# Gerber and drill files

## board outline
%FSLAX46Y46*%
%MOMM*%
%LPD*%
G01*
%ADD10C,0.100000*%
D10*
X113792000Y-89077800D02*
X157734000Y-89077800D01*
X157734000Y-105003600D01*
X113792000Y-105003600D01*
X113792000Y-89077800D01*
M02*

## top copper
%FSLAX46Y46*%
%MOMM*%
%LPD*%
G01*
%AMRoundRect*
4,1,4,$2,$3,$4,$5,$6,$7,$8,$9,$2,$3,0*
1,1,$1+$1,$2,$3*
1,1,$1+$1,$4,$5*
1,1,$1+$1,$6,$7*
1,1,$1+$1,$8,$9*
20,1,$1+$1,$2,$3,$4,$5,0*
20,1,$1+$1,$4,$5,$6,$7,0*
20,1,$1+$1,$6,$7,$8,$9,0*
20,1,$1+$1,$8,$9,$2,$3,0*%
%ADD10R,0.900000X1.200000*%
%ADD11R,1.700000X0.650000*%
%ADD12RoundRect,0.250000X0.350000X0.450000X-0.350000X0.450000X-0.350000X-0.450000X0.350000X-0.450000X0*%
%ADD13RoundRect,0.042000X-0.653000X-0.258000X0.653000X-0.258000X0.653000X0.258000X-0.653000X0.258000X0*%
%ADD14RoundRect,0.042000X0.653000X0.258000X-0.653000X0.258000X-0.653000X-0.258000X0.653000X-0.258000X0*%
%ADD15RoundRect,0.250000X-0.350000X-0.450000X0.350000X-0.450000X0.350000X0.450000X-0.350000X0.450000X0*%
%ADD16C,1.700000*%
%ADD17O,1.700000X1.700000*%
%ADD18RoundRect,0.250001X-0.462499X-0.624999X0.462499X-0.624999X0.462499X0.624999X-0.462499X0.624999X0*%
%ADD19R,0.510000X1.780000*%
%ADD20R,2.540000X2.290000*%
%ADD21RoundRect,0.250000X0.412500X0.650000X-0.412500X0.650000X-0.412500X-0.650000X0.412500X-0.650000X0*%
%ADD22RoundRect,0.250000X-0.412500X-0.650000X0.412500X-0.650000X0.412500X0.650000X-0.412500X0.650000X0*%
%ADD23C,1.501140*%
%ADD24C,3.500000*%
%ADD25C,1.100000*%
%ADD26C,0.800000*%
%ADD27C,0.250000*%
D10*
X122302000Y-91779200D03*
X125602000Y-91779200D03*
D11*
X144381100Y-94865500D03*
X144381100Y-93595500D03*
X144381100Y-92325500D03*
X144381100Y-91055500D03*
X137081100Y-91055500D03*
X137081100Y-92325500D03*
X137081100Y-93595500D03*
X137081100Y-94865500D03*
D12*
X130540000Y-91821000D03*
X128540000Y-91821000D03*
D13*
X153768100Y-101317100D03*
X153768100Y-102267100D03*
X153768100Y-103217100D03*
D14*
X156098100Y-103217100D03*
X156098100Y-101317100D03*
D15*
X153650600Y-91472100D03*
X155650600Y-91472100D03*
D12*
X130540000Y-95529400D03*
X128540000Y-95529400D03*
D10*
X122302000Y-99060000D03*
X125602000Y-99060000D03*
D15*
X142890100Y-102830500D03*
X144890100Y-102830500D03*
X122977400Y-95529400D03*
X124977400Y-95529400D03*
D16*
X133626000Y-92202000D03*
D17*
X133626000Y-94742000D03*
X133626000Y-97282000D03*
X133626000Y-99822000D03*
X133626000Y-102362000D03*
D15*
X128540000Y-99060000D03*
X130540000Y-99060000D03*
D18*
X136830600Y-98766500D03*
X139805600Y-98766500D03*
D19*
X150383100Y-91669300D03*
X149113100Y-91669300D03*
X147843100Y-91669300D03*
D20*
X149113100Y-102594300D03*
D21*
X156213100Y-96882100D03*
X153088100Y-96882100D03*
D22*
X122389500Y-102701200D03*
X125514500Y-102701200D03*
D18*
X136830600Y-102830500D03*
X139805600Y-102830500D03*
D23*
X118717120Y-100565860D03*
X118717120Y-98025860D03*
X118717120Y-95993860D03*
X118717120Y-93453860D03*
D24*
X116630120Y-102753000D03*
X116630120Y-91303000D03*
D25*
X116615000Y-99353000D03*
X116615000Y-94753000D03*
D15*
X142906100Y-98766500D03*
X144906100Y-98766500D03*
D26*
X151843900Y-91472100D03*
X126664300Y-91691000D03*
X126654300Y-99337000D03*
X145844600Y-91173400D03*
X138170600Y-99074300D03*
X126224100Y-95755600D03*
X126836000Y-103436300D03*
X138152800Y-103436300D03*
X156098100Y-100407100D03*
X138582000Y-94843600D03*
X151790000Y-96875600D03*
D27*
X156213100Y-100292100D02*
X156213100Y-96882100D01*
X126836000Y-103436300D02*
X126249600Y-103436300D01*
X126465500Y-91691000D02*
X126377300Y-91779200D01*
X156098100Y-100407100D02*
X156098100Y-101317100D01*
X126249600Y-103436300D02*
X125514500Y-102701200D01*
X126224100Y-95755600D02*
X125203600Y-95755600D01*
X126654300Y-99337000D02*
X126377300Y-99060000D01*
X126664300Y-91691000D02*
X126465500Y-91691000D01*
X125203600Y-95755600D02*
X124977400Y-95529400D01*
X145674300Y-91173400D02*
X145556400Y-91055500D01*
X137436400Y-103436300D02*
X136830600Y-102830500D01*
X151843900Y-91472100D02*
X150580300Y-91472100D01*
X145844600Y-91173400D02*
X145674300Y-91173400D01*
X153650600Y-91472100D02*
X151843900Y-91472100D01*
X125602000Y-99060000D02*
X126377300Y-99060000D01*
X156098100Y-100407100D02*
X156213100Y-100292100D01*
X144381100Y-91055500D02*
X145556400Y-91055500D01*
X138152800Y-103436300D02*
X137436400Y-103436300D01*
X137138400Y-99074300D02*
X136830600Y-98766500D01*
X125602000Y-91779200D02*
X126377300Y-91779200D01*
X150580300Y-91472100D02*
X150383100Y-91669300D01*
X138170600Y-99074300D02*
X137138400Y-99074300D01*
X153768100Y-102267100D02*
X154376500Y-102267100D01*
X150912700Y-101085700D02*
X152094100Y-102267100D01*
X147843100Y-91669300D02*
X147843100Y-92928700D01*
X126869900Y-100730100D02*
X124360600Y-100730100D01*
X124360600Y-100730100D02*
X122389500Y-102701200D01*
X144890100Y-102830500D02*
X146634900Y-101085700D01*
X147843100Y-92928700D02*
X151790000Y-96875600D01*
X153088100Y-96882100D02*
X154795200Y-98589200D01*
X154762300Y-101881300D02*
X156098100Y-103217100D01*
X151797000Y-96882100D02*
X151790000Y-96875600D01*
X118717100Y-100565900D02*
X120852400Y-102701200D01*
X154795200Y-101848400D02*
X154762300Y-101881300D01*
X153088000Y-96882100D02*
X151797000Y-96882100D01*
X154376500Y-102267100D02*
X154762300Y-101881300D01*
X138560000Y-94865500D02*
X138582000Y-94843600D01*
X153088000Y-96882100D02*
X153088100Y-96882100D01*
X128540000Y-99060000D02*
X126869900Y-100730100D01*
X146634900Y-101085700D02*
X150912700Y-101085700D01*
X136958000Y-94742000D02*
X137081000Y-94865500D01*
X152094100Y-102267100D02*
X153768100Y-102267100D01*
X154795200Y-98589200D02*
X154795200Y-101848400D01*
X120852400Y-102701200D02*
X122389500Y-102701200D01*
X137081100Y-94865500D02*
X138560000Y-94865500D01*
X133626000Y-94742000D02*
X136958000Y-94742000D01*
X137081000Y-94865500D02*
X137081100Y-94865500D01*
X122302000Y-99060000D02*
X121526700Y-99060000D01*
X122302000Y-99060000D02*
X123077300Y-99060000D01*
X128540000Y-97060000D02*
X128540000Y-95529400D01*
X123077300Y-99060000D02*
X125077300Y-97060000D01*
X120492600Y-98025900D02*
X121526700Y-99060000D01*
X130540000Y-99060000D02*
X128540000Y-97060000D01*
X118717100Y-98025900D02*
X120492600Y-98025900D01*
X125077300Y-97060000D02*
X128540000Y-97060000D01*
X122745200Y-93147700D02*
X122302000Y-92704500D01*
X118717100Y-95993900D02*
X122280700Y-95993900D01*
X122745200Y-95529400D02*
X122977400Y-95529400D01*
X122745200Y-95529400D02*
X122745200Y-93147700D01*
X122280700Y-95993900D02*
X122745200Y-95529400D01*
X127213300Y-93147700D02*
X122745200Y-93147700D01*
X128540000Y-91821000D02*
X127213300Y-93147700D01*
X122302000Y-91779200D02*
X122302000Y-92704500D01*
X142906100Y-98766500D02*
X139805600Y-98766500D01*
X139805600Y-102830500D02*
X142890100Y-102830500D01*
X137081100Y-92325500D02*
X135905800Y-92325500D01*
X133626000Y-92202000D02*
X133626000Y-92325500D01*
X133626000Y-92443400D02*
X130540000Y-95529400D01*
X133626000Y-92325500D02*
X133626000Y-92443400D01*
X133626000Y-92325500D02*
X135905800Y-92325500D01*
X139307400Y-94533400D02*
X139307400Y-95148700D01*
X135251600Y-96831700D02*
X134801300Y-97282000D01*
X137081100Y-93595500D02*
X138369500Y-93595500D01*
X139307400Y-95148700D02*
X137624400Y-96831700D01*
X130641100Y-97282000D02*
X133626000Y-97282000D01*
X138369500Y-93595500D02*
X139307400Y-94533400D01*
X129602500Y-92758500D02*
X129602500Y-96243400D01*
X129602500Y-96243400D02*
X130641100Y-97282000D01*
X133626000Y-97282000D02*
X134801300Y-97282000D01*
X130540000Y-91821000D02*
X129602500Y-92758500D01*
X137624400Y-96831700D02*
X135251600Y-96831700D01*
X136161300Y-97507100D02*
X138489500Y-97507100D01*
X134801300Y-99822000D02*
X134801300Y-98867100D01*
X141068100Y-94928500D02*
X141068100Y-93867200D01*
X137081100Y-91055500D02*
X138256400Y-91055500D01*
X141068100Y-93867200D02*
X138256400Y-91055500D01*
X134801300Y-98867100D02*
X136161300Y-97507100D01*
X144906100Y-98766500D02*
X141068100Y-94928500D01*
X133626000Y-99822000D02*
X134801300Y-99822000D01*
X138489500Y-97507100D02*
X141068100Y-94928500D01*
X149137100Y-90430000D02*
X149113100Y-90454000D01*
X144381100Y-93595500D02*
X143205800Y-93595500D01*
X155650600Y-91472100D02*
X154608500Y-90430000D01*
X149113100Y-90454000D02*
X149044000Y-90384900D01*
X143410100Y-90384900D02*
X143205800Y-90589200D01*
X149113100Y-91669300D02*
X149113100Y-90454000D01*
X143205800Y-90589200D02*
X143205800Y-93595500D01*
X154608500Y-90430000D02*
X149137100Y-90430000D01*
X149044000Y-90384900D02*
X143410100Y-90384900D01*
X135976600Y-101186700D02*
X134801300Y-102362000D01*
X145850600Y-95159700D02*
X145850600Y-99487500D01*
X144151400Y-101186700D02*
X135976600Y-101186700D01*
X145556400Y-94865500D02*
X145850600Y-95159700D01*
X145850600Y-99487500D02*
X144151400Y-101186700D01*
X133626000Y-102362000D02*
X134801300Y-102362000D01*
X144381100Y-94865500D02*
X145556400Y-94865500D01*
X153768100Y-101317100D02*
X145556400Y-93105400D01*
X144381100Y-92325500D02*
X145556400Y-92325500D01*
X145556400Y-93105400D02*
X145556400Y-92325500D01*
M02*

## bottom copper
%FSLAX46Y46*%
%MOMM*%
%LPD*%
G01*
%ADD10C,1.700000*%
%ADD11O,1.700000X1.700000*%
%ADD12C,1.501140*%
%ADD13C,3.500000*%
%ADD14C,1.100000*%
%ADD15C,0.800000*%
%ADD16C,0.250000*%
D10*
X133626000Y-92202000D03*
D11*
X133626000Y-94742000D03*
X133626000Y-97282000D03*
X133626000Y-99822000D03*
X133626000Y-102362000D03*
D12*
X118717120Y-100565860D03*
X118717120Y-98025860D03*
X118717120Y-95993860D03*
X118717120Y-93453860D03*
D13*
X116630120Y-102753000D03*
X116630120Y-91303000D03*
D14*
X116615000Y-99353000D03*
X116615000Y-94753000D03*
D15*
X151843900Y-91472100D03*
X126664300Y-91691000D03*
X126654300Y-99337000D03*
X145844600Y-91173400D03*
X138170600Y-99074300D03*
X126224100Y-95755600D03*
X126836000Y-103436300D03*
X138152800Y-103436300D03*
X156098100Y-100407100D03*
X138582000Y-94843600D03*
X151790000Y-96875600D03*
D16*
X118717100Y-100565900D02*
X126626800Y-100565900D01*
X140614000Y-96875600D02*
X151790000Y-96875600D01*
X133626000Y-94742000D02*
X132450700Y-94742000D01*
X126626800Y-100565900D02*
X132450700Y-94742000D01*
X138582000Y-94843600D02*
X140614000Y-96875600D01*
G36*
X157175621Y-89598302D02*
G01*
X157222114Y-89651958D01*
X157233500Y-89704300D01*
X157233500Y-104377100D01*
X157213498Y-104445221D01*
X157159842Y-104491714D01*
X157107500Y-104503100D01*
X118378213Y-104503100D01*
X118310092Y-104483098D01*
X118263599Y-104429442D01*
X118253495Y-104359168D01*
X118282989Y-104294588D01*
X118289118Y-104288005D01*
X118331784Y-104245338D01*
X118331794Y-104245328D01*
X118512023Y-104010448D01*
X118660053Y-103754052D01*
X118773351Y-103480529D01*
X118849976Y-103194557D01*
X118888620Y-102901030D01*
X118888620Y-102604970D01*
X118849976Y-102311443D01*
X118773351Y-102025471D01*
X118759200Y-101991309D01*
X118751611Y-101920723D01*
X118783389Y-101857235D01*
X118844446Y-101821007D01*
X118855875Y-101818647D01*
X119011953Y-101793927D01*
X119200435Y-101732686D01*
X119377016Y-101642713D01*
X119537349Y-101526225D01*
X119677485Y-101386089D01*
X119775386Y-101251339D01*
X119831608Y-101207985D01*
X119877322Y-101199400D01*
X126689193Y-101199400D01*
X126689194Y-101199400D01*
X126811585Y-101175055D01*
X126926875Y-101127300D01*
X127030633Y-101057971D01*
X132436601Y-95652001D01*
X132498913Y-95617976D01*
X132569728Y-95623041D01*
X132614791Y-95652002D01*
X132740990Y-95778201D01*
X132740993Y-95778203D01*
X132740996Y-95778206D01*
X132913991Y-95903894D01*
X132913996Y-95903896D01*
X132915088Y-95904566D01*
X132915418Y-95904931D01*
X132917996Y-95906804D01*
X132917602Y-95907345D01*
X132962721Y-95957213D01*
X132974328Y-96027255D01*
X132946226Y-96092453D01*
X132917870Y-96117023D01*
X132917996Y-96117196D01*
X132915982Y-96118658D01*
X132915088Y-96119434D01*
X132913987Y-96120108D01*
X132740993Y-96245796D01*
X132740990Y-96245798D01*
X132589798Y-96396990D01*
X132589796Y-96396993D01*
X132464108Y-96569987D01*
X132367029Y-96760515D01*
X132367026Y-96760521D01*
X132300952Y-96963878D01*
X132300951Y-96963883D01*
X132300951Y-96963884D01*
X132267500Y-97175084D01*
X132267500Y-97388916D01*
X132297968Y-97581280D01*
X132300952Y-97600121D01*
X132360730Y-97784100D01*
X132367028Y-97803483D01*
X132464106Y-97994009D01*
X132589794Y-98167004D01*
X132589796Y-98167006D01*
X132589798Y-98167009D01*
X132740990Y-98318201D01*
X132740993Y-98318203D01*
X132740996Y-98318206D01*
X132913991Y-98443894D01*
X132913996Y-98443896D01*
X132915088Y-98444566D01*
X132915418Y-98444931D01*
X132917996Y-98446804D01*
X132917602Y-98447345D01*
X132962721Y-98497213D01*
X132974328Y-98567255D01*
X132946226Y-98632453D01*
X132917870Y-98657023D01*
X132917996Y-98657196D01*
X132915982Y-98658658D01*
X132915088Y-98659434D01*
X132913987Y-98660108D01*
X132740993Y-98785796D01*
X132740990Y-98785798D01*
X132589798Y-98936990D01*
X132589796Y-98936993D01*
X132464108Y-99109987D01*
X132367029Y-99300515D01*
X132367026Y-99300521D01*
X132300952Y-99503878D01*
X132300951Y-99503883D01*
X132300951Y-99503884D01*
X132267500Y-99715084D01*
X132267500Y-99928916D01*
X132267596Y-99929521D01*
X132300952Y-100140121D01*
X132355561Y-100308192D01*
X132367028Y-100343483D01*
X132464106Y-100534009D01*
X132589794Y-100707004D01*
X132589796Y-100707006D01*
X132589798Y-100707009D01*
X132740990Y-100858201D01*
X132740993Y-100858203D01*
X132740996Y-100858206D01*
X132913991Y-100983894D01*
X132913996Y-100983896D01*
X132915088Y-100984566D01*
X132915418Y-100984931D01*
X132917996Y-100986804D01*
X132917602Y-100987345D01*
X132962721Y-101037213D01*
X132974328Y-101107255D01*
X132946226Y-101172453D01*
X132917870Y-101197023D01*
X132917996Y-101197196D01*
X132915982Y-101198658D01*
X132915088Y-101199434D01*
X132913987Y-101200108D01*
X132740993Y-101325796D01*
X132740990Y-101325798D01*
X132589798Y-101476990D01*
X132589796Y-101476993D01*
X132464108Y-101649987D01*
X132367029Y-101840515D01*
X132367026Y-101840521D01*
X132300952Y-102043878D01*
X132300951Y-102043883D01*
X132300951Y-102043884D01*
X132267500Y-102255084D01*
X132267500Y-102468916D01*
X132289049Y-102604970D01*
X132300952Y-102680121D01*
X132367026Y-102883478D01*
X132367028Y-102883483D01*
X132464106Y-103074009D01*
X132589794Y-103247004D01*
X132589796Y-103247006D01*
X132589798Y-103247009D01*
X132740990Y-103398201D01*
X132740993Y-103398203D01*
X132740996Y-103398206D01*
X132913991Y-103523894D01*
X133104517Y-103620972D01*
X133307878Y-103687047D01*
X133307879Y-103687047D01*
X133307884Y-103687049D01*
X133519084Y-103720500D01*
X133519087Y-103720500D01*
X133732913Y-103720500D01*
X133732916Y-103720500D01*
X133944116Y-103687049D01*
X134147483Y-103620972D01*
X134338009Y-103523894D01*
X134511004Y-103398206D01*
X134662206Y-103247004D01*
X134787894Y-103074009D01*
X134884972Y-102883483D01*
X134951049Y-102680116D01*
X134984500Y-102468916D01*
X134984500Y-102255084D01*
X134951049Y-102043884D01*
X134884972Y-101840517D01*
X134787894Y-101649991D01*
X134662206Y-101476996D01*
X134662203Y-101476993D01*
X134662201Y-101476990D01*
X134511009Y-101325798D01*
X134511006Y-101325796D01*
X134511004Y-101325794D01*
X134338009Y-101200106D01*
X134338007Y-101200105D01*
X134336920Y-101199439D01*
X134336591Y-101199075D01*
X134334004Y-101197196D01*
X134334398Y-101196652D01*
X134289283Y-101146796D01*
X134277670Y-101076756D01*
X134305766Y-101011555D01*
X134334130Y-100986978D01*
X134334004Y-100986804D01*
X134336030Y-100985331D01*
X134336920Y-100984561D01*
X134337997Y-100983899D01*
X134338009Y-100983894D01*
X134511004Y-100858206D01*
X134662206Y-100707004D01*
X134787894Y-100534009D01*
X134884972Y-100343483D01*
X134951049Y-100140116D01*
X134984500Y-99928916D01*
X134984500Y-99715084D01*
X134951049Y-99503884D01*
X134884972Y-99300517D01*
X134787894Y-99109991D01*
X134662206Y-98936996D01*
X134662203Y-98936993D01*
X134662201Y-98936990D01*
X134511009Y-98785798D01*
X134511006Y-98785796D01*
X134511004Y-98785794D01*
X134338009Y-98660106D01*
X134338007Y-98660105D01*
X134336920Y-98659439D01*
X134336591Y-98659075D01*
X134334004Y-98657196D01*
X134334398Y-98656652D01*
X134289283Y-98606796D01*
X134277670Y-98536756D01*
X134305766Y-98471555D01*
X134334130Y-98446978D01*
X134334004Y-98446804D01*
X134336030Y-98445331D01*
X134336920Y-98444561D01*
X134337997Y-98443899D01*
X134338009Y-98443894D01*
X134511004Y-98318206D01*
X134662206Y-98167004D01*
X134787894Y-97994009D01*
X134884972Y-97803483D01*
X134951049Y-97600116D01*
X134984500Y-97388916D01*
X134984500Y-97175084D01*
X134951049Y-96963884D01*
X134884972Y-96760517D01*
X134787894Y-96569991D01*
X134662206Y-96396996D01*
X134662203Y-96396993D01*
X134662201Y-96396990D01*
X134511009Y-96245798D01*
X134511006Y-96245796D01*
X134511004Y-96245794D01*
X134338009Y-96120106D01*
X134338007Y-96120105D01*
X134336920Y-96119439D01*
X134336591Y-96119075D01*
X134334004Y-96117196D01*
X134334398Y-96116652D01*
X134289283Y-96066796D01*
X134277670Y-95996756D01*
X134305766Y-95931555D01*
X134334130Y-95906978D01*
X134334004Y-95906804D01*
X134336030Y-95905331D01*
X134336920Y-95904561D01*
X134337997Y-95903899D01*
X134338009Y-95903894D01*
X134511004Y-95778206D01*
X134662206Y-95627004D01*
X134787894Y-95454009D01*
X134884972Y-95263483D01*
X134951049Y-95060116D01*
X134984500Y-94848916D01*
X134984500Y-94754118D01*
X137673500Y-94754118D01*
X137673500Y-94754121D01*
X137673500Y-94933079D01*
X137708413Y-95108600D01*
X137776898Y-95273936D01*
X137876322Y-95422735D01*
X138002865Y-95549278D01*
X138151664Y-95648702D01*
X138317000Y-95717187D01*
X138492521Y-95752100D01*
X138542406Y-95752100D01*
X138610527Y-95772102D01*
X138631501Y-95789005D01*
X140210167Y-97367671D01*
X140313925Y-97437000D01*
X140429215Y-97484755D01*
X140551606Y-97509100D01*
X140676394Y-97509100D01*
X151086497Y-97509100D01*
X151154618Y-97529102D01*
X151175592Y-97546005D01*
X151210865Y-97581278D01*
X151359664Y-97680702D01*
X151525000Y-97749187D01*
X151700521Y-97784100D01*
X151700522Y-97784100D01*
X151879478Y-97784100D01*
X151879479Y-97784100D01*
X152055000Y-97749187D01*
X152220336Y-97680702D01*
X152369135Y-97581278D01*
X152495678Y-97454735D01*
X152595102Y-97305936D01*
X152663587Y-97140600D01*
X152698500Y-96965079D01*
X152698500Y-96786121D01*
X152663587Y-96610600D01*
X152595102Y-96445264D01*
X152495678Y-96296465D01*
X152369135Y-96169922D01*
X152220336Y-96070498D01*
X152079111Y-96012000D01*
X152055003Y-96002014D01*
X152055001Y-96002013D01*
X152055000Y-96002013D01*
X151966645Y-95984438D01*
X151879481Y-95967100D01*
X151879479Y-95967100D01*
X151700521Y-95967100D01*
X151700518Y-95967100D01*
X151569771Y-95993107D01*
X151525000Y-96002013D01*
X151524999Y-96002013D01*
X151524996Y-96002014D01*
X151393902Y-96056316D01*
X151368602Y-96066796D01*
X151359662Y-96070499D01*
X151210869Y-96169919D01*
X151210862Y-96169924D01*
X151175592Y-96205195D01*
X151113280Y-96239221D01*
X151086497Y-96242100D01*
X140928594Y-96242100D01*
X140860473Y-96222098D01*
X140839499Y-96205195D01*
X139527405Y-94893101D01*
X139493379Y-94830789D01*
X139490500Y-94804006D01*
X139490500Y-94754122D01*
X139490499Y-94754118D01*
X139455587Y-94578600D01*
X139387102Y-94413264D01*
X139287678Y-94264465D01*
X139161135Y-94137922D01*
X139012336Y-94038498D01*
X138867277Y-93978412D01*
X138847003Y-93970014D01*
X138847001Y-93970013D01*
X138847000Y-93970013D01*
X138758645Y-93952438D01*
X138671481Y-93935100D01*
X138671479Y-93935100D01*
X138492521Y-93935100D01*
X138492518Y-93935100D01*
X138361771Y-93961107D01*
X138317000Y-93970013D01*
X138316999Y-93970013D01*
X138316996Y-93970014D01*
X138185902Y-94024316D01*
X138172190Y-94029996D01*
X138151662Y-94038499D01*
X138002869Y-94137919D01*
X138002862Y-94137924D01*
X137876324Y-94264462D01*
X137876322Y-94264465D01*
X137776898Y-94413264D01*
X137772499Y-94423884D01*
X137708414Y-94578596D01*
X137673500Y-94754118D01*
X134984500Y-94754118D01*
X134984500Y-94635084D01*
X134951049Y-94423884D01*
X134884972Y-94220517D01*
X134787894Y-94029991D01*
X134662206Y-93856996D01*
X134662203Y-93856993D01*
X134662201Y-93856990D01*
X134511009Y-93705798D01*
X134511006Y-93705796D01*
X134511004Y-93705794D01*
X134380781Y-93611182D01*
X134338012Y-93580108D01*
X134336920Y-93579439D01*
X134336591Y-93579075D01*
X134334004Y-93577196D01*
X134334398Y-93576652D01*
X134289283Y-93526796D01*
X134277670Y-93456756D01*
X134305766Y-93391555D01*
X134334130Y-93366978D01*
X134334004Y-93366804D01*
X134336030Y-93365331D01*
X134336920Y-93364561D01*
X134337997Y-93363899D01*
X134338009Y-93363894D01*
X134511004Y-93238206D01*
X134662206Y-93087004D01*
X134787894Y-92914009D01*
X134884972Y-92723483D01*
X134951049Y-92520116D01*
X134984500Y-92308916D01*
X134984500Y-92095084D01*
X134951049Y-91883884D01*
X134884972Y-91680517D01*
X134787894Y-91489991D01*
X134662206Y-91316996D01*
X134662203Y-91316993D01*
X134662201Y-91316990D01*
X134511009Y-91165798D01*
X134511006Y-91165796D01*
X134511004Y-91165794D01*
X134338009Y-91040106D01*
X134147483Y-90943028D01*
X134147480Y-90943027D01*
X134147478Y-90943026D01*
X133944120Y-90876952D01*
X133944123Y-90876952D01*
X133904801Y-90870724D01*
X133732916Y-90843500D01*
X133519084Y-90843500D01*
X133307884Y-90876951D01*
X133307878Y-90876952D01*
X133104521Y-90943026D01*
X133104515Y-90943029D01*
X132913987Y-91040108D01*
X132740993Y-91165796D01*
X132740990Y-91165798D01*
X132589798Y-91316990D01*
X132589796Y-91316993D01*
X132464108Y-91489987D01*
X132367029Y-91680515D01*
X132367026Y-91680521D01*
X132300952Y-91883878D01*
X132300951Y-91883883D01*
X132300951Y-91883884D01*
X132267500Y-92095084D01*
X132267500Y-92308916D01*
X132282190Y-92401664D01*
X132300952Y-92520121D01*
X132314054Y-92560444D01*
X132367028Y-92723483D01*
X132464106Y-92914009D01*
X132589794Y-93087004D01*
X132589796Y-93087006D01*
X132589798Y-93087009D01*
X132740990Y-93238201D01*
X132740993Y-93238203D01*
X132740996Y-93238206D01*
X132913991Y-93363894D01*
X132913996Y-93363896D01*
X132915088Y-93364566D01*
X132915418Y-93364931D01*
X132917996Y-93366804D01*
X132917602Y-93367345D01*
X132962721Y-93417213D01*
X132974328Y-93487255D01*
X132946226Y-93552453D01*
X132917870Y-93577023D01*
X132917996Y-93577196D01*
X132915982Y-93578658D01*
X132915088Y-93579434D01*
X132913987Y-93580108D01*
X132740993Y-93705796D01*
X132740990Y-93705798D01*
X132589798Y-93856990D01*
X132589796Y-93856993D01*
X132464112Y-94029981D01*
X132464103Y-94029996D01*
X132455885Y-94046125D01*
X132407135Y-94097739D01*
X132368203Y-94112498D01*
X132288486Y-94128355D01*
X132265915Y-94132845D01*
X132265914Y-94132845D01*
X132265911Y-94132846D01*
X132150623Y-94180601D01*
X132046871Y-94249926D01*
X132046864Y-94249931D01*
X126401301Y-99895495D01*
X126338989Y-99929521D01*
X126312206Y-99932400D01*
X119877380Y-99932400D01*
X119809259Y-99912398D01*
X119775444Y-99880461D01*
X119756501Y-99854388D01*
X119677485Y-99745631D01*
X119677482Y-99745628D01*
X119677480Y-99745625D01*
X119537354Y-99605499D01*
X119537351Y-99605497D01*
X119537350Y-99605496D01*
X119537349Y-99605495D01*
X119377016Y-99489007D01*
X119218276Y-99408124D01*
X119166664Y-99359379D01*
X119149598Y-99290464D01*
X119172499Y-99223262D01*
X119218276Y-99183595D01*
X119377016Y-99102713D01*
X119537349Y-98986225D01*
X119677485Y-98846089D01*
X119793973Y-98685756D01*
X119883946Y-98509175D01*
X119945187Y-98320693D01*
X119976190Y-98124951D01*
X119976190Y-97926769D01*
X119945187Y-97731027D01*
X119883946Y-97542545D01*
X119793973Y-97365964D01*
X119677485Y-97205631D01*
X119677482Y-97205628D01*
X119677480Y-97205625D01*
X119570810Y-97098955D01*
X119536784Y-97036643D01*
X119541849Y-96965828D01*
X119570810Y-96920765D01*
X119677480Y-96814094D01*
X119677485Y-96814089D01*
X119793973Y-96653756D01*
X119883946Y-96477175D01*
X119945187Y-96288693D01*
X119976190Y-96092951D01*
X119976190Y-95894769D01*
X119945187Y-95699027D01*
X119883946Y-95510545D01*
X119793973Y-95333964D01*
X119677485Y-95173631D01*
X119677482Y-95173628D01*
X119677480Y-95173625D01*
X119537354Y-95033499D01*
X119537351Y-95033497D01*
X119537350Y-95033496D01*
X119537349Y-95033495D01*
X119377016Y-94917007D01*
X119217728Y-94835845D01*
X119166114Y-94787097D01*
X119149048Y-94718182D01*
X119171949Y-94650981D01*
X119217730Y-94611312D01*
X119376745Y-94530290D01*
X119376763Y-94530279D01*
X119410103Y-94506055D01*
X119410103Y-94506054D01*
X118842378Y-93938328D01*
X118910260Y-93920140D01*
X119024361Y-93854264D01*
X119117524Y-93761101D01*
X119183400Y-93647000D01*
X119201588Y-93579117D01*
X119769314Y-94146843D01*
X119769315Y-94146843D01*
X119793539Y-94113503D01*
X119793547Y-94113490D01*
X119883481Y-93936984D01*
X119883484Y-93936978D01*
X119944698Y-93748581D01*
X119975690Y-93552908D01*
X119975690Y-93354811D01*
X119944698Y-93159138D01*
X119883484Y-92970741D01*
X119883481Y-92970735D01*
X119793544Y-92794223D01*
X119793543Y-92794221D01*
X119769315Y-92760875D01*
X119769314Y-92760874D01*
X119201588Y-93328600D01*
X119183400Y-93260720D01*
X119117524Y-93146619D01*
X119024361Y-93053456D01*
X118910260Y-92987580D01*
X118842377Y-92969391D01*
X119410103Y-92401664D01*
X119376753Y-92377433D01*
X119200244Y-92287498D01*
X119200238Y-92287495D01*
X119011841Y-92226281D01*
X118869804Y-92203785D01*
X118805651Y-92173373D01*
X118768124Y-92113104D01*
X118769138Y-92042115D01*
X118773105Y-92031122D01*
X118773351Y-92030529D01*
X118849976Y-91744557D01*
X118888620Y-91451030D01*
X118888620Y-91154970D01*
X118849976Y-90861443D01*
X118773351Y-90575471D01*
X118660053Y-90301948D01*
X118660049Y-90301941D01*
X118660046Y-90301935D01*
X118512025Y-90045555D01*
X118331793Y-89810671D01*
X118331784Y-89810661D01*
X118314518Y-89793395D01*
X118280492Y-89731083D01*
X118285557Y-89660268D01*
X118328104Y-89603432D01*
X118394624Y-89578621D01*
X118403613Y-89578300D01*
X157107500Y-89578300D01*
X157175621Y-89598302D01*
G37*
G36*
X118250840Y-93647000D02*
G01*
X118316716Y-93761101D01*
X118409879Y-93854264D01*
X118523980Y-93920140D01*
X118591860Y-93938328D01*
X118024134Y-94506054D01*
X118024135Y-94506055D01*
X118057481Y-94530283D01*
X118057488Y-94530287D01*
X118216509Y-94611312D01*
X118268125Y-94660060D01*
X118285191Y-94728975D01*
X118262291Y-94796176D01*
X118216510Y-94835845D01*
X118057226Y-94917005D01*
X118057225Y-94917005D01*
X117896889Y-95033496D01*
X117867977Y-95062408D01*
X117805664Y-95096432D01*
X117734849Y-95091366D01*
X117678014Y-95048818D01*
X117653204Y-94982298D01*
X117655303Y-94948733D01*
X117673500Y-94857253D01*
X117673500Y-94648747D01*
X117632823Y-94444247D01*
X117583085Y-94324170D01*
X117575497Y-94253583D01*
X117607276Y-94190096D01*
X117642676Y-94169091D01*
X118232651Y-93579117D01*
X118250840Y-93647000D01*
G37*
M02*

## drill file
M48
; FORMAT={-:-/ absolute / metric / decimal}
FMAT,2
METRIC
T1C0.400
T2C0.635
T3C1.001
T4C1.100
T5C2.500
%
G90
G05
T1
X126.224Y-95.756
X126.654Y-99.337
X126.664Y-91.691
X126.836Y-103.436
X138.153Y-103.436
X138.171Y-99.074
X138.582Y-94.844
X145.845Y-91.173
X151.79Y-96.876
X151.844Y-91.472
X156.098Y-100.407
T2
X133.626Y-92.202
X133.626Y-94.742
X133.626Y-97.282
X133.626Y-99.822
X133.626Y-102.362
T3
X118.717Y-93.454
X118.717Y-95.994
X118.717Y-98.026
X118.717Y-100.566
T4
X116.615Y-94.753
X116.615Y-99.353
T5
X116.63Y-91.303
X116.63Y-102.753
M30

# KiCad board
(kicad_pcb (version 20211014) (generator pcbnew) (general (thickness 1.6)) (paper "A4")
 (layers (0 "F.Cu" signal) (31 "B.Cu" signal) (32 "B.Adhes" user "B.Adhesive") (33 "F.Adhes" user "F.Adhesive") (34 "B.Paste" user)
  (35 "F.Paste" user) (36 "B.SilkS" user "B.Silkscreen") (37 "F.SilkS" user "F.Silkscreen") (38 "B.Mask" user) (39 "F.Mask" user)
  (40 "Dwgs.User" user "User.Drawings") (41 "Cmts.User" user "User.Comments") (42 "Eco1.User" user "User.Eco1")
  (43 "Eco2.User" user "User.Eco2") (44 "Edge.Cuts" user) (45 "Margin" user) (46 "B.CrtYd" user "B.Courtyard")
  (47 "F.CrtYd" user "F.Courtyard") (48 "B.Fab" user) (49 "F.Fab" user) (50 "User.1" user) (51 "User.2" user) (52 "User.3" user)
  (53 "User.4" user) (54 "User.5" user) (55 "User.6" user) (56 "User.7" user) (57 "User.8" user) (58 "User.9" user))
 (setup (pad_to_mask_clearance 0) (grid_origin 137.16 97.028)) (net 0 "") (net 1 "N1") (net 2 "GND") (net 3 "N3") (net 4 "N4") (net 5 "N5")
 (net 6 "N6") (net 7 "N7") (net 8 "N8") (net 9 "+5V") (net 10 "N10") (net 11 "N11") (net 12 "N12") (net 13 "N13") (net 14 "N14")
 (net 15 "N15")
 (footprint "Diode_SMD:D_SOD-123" (layer "F.Cu") (at 123.952 91.7792)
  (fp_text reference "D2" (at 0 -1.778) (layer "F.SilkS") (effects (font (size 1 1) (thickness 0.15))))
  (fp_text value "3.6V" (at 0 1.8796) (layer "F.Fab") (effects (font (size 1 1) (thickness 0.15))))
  (pad "1" smd rect (at -1.65 0) (size 0.9 1.2) (layers "F.Cu" "F.Paste" "F.Mask") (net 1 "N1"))
  (pad "2" smd rect (at 1.65 0) (size 0.9 1.2) (layers "F.Cu" "F.Paste" "F.Mask") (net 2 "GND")))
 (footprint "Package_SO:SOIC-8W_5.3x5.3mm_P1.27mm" (layer "F.Cu") (at 140.7311 92.9605 180)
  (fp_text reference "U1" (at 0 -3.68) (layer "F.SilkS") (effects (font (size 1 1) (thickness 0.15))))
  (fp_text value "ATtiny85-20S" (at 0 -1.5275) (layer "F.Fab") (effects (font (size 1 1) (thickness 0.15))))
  (pad "1" smd rect (at -3.65 -1.905 180) (size 1.7 0.65) (layers "F.Cu" "F.Paste" "F.Mask") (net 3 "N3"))
  (pad "2" smd rect (at -3.65 -0.635 180) (size 1.7 0.65) (layers "F.Cu" "F.Paste" "F.Mask") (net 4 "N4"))
  (pad "3" smd rect (at -3.65 0.635 180) (size 1.7 0.65) (layers "F.Cu" "F.Paste" "F.Mask") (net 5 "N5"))
  (pad "4" smd rect (at -3.65 1.905 180) (size 1.7 0.65) (layers "F.Cu" "F.Paste" "F.Mask") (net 2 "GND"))
  (pad "5" smd rect (at 3.65 1.905 180) (size 1.7 0.65) (layers "F.Cu" "F.Paste" "F.Mask") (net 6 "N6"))
  (pad "6" smd rect (at 3.65 0.635 180) (size 1.7 0.65) (layers "F.Cu" "F.Paste" "F.Mask") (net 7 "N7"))
  (pad "7" smd rect (at 3.65 -0.635 180) (size 1.7 0.65) (layers "F.Cu" "F.Paste" "F.Mask") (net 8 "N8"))
  (pad "8" smd rect (at 3.65 -1.905 180) (size 1.7 0.65) (layers "F.Cu" "F.Paste" "F.Mask") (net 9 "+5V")))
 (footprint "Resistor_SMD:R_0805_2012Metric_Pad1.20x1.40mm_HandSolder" (layer "F.Cu") (at 129.54 91.821 180)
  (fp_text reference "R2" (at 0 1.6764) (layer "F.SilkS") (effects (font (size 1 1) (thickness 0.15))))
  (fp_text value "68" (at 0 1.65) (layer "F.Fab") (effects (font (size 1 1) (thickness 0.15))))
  (pad "1" smd roundrect (at -1 0 180) (size 1.2 1.4) (layers "F.Cu" "F.Paste" "F.Mask") (roundrect_rratio 0.208333) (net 8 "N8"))
  (pad "2" smd roundrect (at 1 0 180) (size 1.2 1.4) (layers "F.Cu" "F.Paste" "F.Mask") (roundrect_rratio 0.208333) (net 1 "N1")))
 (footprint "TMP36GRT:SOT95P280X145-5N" (layer "F.Cu") (at 154.9331 102.2671)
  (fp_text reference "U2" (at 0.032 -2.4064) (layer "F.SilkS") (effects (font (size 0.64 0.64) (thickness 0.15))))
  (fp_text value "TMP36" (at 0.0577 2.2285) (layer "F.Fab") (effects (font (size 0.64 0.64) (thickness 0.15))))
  (pad "1" smd roundrect locked (at -1.165 -0.95) (size 1.39 0.6) (layers "F.Cu" "F.Paste" "F.Mask") (roundrect_rratio 0.07) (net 5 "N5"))
  (pad "2" smd roundrect locked (at -1.165 0) (size 1.39 0.6) (layers "F.Cu" "F.Paste" "F.Mask") (roundrect_rratio 0.07) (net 9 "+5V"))
  (pad "3" smd roundrect locked (at -1.165 0.95) (size 1.39 0.6) (layers "F.Cu" "F.Paste" "F.Mask") (roundrect_rratio 0.07))
  (pad "4" smd roundrect locked (at 1.165 0.95 180) (size 1.39 0.6) (layers "F.Cu" "F.Paste" "F.Mask") (roundrect_rratio 0.07) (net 9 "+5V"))
  (pad "5" smd roundrect locked (at 1.165 -0.95 180) (size 1.39 0.6) (layers "F.Cu" "F.Paste" "F.Mask") (roundrect_rratio 0.07)
   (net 2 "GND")))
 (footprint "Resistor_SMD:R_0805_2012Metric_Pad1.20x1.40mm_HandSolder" (layer "F.Cu") (at 154.6506 91.4721)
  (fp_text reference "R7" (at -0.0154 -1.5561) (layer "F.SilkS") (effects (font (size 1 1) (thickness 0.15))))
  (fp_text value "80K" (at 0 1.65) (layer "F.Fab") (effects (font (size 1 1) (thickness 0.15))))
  (pad "1" smd roundrect (at -1 0) (size 1.2 1.4) (layers "F.Cu" "F.Paste" "F.Mask") (roundrect_rratio 0.208333) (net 2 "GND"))
  (pad "2" smd roundrect (at 1 0) (size 1.2 1.4) (layers "F.Cu" "F.Paste" "F.Mask") (roundrect_rratio 0.208333) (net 4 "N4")))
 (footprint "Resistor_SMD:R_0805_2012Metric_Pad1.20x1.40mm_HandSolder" (layer "F.Cu") (at 129.54 95.5294 180)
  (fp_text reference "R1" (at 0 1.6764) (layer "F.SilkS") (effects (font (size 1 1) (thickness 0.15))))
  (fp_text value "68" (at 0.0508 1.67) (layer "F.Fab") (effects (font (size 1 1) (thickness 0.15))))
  (pad "1" smd roundrect (at -1 0 180) (size 1.2 1.4) (layers "F.Cu" "F.Paste" "F.Mask") (roundrect_rratio 0.208333) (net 7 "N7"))
  (pad "2" smd roundrect (at 1 0 180) (size 1.2 1.4) (layers "F.Cu" "F.Paste" "F.Mask") (roundrect_rratio 0.208333) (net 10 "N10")))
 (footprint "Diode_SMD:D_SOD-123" (layer "F.Cu") (at 123.952 99.06)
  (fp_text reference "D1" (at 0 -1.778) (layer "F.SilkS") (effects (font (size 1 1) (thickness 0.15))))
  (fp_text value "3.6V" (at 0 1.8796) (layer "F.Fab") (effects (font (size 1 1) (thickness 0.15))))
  (pad "1" smd rect (at -1.65 0) (size 0.9 1.2) (layers "F.Cu" "F.Paste" "F.Mask") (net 10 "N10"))
  (pad "2" smd rect (at 1.65 0) (size 0.9 1.2) (layers "F.Cu" "F.Paste" "F.Mask") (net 2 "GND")))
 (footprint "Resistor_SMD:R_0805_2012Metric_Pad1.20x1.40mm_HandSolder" (layer "F.Cu") (at 143.8901 102.8305)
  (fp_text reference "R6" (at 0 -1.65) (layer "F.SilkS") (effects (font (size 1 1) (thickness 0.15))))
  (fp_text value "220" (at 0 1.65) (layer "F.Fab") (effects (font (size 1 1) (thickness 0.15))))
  (pad "1" smd roundrect (at -1 0) (size 1.2 1.4) (layers "F.Cu" "F.Paste" "F.Mask") (roundrect_rratio 0.208333) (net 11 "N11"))
  (pad "2" smd roundrect (at 1 0) (size 1.2 1.4) (layers "F.Cu" "F.Paste" "F.Mask") (roundrect_rratio 0.208333) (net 9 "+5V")))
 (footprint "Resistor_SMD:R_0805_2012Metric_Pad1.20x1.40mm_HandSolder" (layer "F.Cu") (at 123.9774 95.5294)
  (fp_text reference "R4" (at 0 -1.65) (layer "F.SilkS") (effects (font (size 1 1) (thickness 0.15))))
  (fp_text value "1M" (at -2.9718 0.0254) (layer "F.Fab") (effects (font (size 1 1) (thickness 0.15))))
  (pad "1" smd roundrect (at -1 0) (size 1.2 1.4) (layers "F.Cu" "F.Paste" "F.Mask") (roundrect_rratio 0.208333) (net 1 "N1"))
  (pad "2" smd roundrect (at 1 0) (size 1.2 1.4) (layers "F.Cu" "F.Paste" "F.Mask") (roundrect_rratio 0.208333) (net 2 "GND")))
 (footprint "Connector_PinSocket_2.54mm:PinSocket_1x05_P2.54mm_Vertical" (layer "F.Cu") (at 133.626 92.202)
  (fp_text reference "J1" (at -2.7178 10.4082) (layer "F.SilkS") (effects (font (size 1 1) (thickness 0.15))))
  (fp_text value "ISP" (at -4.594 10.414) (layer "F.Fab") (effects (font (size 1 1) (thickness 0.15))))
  (pad "1" thru_hole circle (at 0 0) (size 1.7 1.7) (drill 0.635) (layers *.Cu *.Mask) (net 7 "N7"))
  (pad "2" thru_hole oval (at 0 2.54) (size 1.7 1.7) (drill 0.635) (layers *.Cu *.Mask) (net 9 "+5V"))
  (pad "3" thru_hole oval (at 0 5.08) (size 1.7 1.7) (drill 0.635) (layers *.Cu *.Mask) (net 8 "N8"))
  (pad "4" thru_hole oval (at 0 7.62) (size 1.7 1.7) (drill 0.635) (layers *.Cu *.Mask) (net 6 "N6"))
  (pad "5" thru_hole oval (at 0 10.16) (size 1.7 1.7) (drill 0.635) (layers *.Cu *.Mask) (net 3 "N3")))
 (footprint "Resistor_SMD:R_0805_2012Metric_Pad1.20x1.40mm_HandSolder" (layer "F.Cu") (at 129.54 99.06)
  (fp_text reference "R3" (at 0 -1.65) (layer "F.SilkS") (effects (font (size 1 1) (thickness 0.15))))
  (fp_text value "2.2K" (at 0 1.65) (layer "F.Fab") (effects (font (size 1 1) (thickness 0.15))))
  (pad "1" smd roundrect (at -1 0) (size 1.2 1.4) (layers "F.Cu" "F.Paste" "F.Mask") (roundrect_rratio 0.208333) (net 9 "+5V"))
  (pad "2" smd roundrect (at 1 0) (size 1.2 1.4) (layers "F.Cu" "F.Paste" "F.Mask") (roundrect_rratio 0.208333) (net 10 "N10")))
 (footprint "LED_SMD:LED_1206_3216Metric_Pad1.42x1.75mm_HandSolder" (layer "F.Cu") (at 138.3181 98.7665)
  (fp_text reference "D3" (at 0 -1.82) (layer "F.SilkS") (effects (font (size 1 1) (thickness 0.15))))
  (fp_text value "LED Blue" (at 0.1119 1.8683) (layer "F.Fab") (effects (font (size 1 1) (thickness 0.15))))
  (pad "1" smd roundrect (at -1.4875 0) (size 1.425 1.75) (layers "F.Cu" "F.Paste" "F.Mask") (roundrect_rratio 0.175439) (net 2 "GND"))
  (pad "2" smd roundrect (at 1.4875 0) (size 1.425 1.75) (layers "F.Cu" "F.Paste" "F.Mask") (roundrect_rratio 0.175439) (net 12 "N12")))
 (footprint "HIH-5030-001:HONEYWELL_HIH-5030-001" (layer "F.Cu") (at 149.1131 97.0043 180)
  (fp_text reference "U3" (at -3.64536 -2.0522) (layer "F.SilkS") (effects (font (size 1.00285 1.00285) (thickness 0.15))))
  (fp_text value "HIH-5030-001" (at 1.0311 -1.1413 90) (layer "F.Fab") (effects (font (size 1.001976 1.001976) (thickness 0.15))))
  (pad "1" smd rect locked (at -1.27 5.335 270) (size 1.78 0.51) (layers "F.Cu" "F.Paste" "F.Mask") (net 2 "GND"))
  (pad "2" smd rect locked (at 0 5.335 270) (size 1.78 0.51) (layers "F.Cu" "F.Paste" "F.Mask") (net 4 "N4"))
  (pad "3" smd rect locked (at 1.27 5.335 270) (size 1.78 0.51) (layers "F.Cu" "F.Paste" "F.Mask") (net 9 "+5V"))
  (pad "4" smd rect locked (at 0 -5.59 180) (size 2.54 2.29) (layers "F.Cu" "F.Paste" "F.Mask") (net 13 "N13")))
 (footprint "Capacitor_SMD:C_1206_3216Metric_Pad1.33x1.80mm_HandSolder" (layer "F.Cu") (at 154.6506 96.8821 180)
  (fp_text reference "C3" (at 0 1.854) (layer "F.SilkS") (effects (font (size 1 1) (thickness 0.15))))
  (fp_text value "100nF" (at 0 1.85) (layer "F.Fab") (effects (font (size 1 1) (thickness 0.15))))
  (pad "1" smd roundrect (at -1.5625 0 180) (size 1.325 1.8) (layers "F.Cu" "F.Paste" "F.Mask") (roundrect_rratio 0.188679) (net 2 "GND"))
  (pad "2" smd roundrect (at 1.5625 0 180) (size 1.325 1.8) (layers "F.Cu" "F.Paste" "F.Mask") (roundrect_rratio 0.188679) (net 9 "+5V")))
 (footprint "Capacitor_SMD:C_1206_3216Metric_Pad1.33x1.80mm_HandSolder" (layer "F.Cu") (at 123.952 102.7012)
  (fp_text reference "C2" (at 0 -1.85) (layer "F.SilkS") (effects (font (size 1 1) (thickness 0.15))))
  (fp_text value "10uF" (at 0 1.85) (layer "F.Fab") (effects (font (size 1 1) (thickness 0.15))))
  (pad "1" smd roundrect (at -1.5625 0) (size 1.325 1.8) (layers "F.Cu" "F.Paste" "F.Mask") (roundrect_rratio 0.188679) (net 9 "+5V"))
  (pad "2" smd roundrect (at 1.5625 0) (size 1.325 1.8) (layers "F.Cu" "F.Paste" "F.Mask") (roundrect_rratio 0.188679) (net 2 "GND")))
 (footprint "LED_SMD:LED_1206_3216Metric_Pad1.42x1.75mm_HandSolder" (layer "F.Cu") (at 138.3181 102.8305)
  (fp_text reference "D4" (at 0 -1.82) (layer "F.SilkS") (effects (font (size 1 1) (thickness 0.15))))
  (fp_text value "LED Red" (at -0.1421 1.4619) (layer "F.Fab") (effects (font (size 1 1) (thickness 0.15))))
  (pad "1" smd roundrect (at -1.4875 0) (size 1.425 1.75) (layers "F.Cu" "F.Paste" "F.Mask") (roundrect_rratio 0.175439) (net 2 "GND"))
  (pad "2" smd roundrect (at 1.4875 0) (size 1.425 1.75) (layers "F.Cu" "F.Paste" "F.Mask") (roundrect_rratio 0.175439) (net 11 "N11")))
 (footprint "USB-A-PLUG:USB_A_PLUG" (layer "F.Cu") (at 118.715 93.453 -90)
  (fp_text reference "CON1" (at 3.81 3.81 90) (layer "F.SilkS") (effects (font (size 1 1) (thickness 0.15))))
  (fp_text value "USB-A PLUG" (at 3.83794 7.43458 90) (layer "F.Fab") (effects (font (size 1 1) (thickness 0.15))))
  (pad "1" thru_hole circle (at 7.11286 -0.00212 180) (size 1.50114 1.50114) (drill 1.00076) (layers *.Cu *.Mask "F.SilkS") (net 9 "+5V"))
  (pad "2" thru_hole circle (at 4.57286 -0.00212 180) (size 1.50114 1.50114) (drill 1.00076) (layers *.Cu *.Mask "F.SilkS") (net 10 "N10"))
  (pad "3" thru_hole circle (at 2.54086 -0.00212 180) (size 1.50114 1.50114) (drill 1.00076) (layers *.Cu *.Mask "F.SilkS") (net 1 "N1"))
  (pad "4" thru_hole circle (at 0.00086 -0.00212 180) (size 1.50114 1.50114) (drill 1.00076) (layers *.Cu *.Mask "F.SilkS") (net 2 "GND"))
  (pad "5" thru_hole circle (at 9.3 2.08488 180) (size 3.5 3.5) (drill 2.5) (layers *.Cu *.Mask "F.SilkS") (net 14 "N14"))
  (pad "6" thru_hole circle (at -2.15 2.08488 180) (size 3.5 3.5) (drill 2.5) (layers *.Cu *.Mask "F.SilkS") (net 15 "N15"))
  (pad "7" thru_hole circle (at 5.9 2.1 180) (size 1.1 1.1) (drill 1.1) (layers *.Cu *.Mask "F.SilkS"))
  (pad "8" thru_hole circle (at 1.3 2.1 180) (size 1.1 1.1) (drill 1.1) (layers *.Cu *.Mask "F.SilkS")))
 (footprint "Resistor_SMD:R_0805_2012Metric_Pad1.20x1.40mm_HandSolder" (layer "F.Cu") (at 143.9061 98.7665)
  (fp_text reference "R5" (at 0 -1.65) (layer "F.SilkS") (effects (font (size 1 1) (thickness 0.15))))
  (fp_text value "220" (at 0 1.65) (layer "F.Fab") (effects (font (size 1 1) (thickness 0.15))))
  (pad "1" smd roundrect (at -1 0) (size 1.2 1.4) (layers "F.Cu" "F.Paste" "F.Mask") (roundrect_rratio 0.208333) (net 12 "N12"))
  (pad "2" smd roundrect (at 1 0) (size 1.2 1.4) (layers "F.Cu" "F.Paste" "F.Mask") (roundrect_rratio 0.208333) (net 6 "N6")))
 (gr_rect (start 113.792 89.0778) (end 157.734 105.0036) (layer "Edge.Cuts") (width 0.1) (fill none))
 (segment (start 156.2131 100.2921) (end 156.2131 96.8821) (width 0.25) (layer "F.Cu") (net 2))
 (segment (start 126.836 103.4363) (end 126.2496 103.4363) (width 0.25) (layer "F.Cu") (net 2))
 (segment (start 126.4655 91.691) (end 126.3773 91.7792) (width 0.25) (layer "F.Cu") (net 2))
 (segment (start 156.0981 100.4071) (end 156.0981 101.3171) (width 0.25) (layer "F.Cu") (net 2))
 (segment (start 126.2496 103.4363) (end 125.5145 102.7012) (width 0.25) (layer "F.Cu") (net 2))
 (segment (start 126.2241 95.7556) (end 125.2036 95.7556) (width 0.25) (layer "F.Cu") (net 2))
 (segment (start 126.6543 99.337) (end 126.3773 99.06) (width 0.25) (layer "F.Cu") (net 2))
 (segment (start 126.6643 91.691) (end 126.4655 91.691) (width 0.25) (layer "F.Cu") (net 2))
 (segment (start 125.2036 95.7556) (end 124.9774 95.5294) (width 0.25) (layer "F.Cu") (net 2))
 (segment (start 145.6743 91.1734) (end 145.5564 91.0555) (width 0.25) (layer "F.Cu") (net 2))
 (segment (start 137.4364 103.4363) (end 136.8306 102.8305) (width 0.25) (layer "F.Cu") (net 2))
 (segment (start 151.8439 91.4721) (end 150.5803 91.4721) (width 0.25) (layer "F.Cu") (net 2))
 (segment (start 145.8446 91.1734) (end 145.6743 91.1734) (width 0.25) (layer "F.Cu") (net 2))
 (segment (start 153.6506 91.4721) (end 151.8439 91.4721) (width 0.25) (layer "F.Cu") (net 2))
 (segment (start 125.602 99.06) (end 126.3773 99.06) (width 0.25) (layer "F.Cu") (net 2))
 (segment (start 156.0981 100.4071) (end 156.2131 100.2921) (width 0.25) (layer "F.Cu") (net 2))
 (segment (start 144.3811 91.0555) (end 145.5564 91.0555) (width 0.25) (layer "F.Cu") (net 2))
 (segment (start 138.1528 103.4363) (end 137.4364 103.4363) (width 0.25) (layer "F.Cu") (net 2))
 (segment (start 137.1384 99.0743) (end 136.8306 98.7665) (width 0.25) (layer "F.Cu") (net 2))
 (segment (start 125.602 91.7792) (end 126.3773 91.7792) (width 0.25) (layer "F.Cu") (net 2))
 (segment (start 150.5803 91.4721) (end 150.3831 91.6693) (width 0.25) (layer "F.Cu") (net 2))
 (segment (start 138.1706 99.0743) (end 137.1384 99.0743) (width 0.25) (layer "F.Cu") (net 2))
 (via (at 151.8439 91.4721) (size 0.8) (drill 0.4) (layers "F.Cu" "B.Cu") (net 2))
 (via (at 126.6643 91.691) (size 0.8) (drill 0.4) (layers "F.Cu" "B.Cu") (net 2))
 (via (at 126.6543 99.337) (size 0.8) (drill 0.4) (layers "F.Cu" "B.Cu") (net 2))
 (via (at 145.8446 91.1734) (size 0.8) (drill 0.4) (layers "F.Cu" "B.Cu") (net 2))
 (via (at 138.1706 99.0743) (size 0.8) (drill 0.4) (layers "F.Cu" "B.Cu") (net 2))
 (via (at 126.2241 95.7556) (size 0.8) (drill 0.4) (layers "F.Cu" "B.Cu") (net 2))
 (via (at 126.836 103.4363) (size 0.8) (drill 0.4) (layers "F.Cu" "B.Cu") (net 2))
 (via (at 138.1528 103.4363) (size 0.8) (drill 0.4) (layers "F.Cu" "B.Cu") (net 2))
 (via (at 156.0981 100.4071) (size 0.8) (drill 0.4) (layers "F.Cu" "B.Cu") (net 2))
 (segment (start 153.7681 102.2671) (end 154.3765 102.2671) (width 0.25) (layer "F.Cu") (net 9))
 (segment (start 150.9127 101.0857) (end 152.0941 102.2671) (width 0.25) (layer "F.Cu") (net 9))
 (segment (start 147.8431 91.6693) (end 147.8431 92.9287) (width 0.25) (layer "F.Cu") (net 9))
 (segment (start 126.8699 100.7301) (end 124.3606 100.7301) (width 0.25) (layer "F.Cu") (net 9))
 (segment (start 124.3606 100.7301) (end 122.3895 102.7012) (width 0.25) (layer "F.Cu") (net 9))
 (segment (start 144.8901 102.8305) (end 146.6349 101.0857) (width 0.25) (layer "F.Cu") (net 9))
 (segment (start 147.8431 92.9287) (end 151.79 96.8756) (width 0.25) (layer "F.Cu") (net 9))
 (segment (start 153.0881 96.8821) (end 154.7952 98.5892) (width 0.25) (layer "F.Cu") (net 9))
 (segment (start 154.7623 101.8813) (end 156.0981 103.2171) (width 0.25) (layer "F.Cu") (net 9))
 (segment (start 151.797 96.8821) (end 151.79 96.8756) (width 0.25) (layer "F.Cu") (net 9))
 (segment (start 118.7171 100.5659) (end 120.8524 102.7012) (width 0.25) (layer "F.Cu") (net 9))
 (segment (start 154.7952 101.8484) (end 154.7623 101.8813) (width 0.25) (layer "F.Cu") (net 9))
 (segment (start 153.088 96.8821) (end 151.797 96.8821) (width 0.25) (layer "F.Cu") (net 9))
 (segment (start 154.3765 102.2671) (end 154.7623 101.8813) (width 0.25) (layer "F.Cu") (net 9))
 (segment (start 138.56 94.8655) (end 138.582 94.8436) (width 0.25) (layer "F.Cu") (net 9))
 (segment (start 153.088 96.8821) (end 153.0881 96.8821) (width 0.25) (layer "F.Cu") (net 9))
 (segment (start 128.54 99.06) (end 126.8699 100.7301) (width 0.25) (layer "F.Cu") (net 9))
 (segment (start 146.6349 101.0857) (end 150.9127 101.0857) (width 0.25) (layer "F.Cu") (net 9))
 (segment (start 136.958 94.742) (end 137.081 94.8655) (width 0.25) (layer "F.Cu") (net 9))
 (segment (start 152.0941 102.2671) (end 153.7681 102.2671) (width 0.25) (layer "F.Cu") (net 9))
 (segment (start 154.7952 98.5892) (end 154.7952 101.8484) (width 0.25) (layer "F.Cu") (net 9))
 (segment (start 120.8524 102.7012) (end 122.3895 102.7012) (width 0.25) (layer "F.Cu") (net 9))
 (segment (start 137.0811 94.8655) (end 138.56 94.8655) (width 0.25) (layer "F.Cu") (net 9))
 (segment (start 133.626 94.742) (end 136.958 94.742) (width 0.25) (layer "F.Cu") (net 9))
 (segment (start 137.081 94.8655) (end 137.0811 94.8655) (width 0.25) (layer "F.Cu") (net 9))
 (via (at 138.582 94.8436) (size 0.8) (drill 0.4) (layers "F.Cu" "B.Cu") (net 9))
 (via (at 151.79 96.8756) (size 0.8) (drill 0.4) (layers "F.Cu" "B.Cu") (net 9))
 (segment (start 118.7171 100.5659) (end 126.6268 100.5659) (width 0.25) (layer "B.Cu") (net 9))
 (segment (start 140.614 96.8756) (end 151.79 96.8756) (width 0.25) (layer "B.Cu") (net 9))
 (segment (start 133.626 94.742) (end 132.4507 94.742) (width 0.25) (layer "B.Cu") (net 9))
 (segment (start 126.6268 100.5659) (end 132.4507 94.742) (width 0.25) (layer "B.Cu") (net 9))
 (segment (start 138.582 94.8436) (end 140.614 96.8756) (width 0.25) (layer "B.Cu") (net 9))
 (segment (start 122.302 99.06) (end 121.5267 99.06) (width 0.25) (layer "F.Cu") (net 10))
 (segment (start 122.302 99.06) (end 123.0773 99.06) (width 0.25) (layer "F.Cu") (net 10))
 (segment (start 128.54 97.06) (end 128.54 95.5294) (width 0.25) (layer "F.Cu") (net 10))
 (segment (start 123.0773 99.06) (end 125.0773 97.06) (width 0.25) (layer "F.Cu") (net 10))
 (segment (start 120.4926 98.0259) (end 121.5267 99.06) (width 0.25) (layer "F.Cu") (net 10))
 (segment (start 130.54 99.06) (end 128.54 97.06) (width 0.25) (layer "F.Cu") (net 10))
 (segment (start 118.7171 98.0259) (end 120.4926 98.0259) (width 0.25) (layer "F.Cu") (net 10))
 (segment (start 125.0773 97.06) (end 128.54 97.06) (width 0.25) (layer "F.Cu") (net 10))
 (segment (start 122.7452 93.1477) (end 122.302 92.7045) (width 0.25) (layer "F.Cu") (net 1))
 (segment (start 118.7171 95.9939) (end 122.2807 95.9939) (width 0.25) (layer "F.Cu") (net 1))
 (segment (start 122.7452 95.5294) (end 122.9774 95.5294) (width 0.25) (layer "F.Cu") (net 1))
 (segment (start 122.7452 95.5294) (end 122.7452 93.1477) (width 0.25) (layer "F.Cu") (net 1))
 (segment (start 122.2807 95.9939) (end 122.7452 95.5294) (width 0.25) (layer "F.Cu") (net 1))
 (segment (start 127.2133 93.1477) (end 122.7452 93.1477) (width 0.25) (layer "F.Cu") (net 1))
 (segment (start 128.54 91.821) (end 127.2133 93.1477) (width 0.25) (layer "F.Cu") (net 1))
 (segment (start 122.302 91.7792) (end 122.302 92.7045) (width 0.25) (layer "F.Cu") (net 1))
 (segment (start 142.9061 98.7665) (end 139.8056 98.7665) (width 0.25) (layer "F.Cu") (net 12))
 (segment (start 139.8056 102.8305) (end 142.8901 102.8305) (width 0.25) (layer "F.Cu") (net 11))
 (segment (start 137.0811 92.3255) (end 135.9058 92.3255) (width 0.25) (layer "F.Cu") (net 7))
 (segment (start 133.626 92.202) (end 133.626 92.3255) (width 0.25) (layer "F.Cu") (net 7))
 (segment (start 133.626 92.4434) (end 130.54 95.5294) (width 0.25) (layer "F.Cu") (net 7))
 (segment (start 133.626 92.3255) (end 133.626 92.4434) (width 0.25) (layer "F.Cu") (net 7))
 (segment (start 133.626 92.3255) (end 135.9058 92.3255) (width 0.25) (layer "F.Cu") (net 7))
 (segment (start 139.3074 94.5334) (end 139.3074 95.1487) (width 0.25) (layer "F.Cu") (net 8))
 (segment (start 135.2516 96.8317) (end 134.8013 97.282) (width 0.25) (layer "F.Cu") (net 8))
 (segment (start 137.0811 93.5955) (end 138.3695 93.5955) (width 0.25) (layer "F.Cu") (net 8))
 (segment (start 139.3074 95.1487) (end 137.6244 96.8317) (width 0.25) (layer "F.Cu") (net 8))
 (segment (start 130.6411 97.282) (end 133.626 97.282) (width 0.25) (layer "F.Cu") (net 8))
 (segment (start 138.3695 93.5955) (end 139.3074 94.5334) (width 0.25) (layer "F.Cu") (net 8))
 (segment (start 129.6025 92.7585) (end 129.6025 96.2434) (width 0.25) (layer "F.Cu") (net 8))
 (segment (start 129.6025 96.2434) (end 130.6411 97.282) (width 0.25) (layer "F.Cu") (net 8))
 (segment (start 133.626 97.282) (end 134.8013 97.282) (width 0.25) (layer "F.Cu") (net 8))
 (segment (start 130.54 91.821) (end 129.6025 92.7585) (width 0.25) (layer "F.Cu") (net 8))
 (segment (start 137.6244 96.8317) (end 135.2516 96.8317) (width 0.25) (layer "F.Cu") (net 8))
 (segment (start 136.1613 97.5071) (end 138.4895 97.5071) (width 0.25) (layer "F.Cu") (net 6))
 (segment (start 134.8013 99.822) (end 134.8013 98.8671) (width 0.25) (layer "F.Cu") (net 6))
 (segment (start 141.0681 94.9285) (end 141.0681 93.8672) (width 0.25) (layer "F.Cu") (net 6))
 (segment (start 137.0811 91.0555) (end 138.2564 91.0555) (width 0.25) (layer "F.Cu") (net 6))
 (segment (start 141.0681 93.8672) (end 138.2564 91.0555) (width 0.25) (layer "F.Cu") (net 6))
 (segment (start 134.8013 98.8671) (end 136.1613 97.5071) (width 0.25) (layer "F.Cu") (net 6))
 (segment (start 144.9061 98.7665) (end 141.0681 94.9285) (width 0.25) (layer "F.Cu") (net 6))
 (segment (start 133.626 99.822) (end 134.8013 99.822) (width 0.25) (layer "F.Cu") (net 6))
 (segment (start 138.4895 97.5071) (end 141.0681 94.9285) (width 0.25) (layer "F.Cu") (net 6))
 (segment (start 149.1371 90.43) (end 149.1131 90.454) (width 0.25) (layer "F.Cu") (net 4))
 (segment (start 144.3811 93.5955) (end 143.2058 93.5955) (width 0.25) (layer "F.Cu") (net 4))
 (segment (start 155.6506 91.4721) (end 154.6085 90.43) (width 0.25) (layer "F.Cu") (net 4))
 (segment (start 149.1131 90.454) (end 149.044 90.3849) (width 0.25) (layer "F.Cu") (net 4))
 (segment (start 143.4101 90.3849) (end 143.2058 90.5892) (width 0.25) (layer "F.Cu") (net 4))
 (segment (start 149.1131 91.6693) (end 149.1131 90.454) (width 0.25) (layer "F.Cu") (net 4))
 (segment (start 143.2058 90.5892) (end 143.2058 93.5955) (width 0.25) (layer "F.Cu") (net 4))
 (segment (start 154.6085 90.43) (end 149.1371 90.43) (width 0.25) (layer "F.Cu") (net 4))
 (segment (start 149.044 90.3849) (end 143.4101 90.3849) (width 0.25) (layer "F.Cu") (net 4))
 (segment (start 135.9766 101.1867) (end 134.8013 102.362) (width 0.25) (layer "F.Cu") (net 3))
 (segment (start 145.8506 95.1597) (end 145.8506 99.4875) (width 0.25) (layer "F.Cu") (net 3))
 (segment (start 144.1514 101.1867) (end 135.9766 101.1867) (width 0.25) (layer "F.Cu") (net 3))
 (segment (start 145.5564 94.8655) (end 145.8506 95.1597) (width 0.25) (layer "F.Cu") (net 3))
 (segment (start 145.8506 99.4875) (end 144.1514 101.1867) (width 0.25) (layer "F.Cu") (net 3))
 (segment (start 133.626 102.362) (end 134.8013 102.362) (width 0.25) (layer "F.Cu") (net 3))
 (segment (start 144.3811 94.8655) (end 145.5564 94.8655) (width 0.25) (layer "F.Cu") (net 3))
 (segment (start 153.7681 101.3171) (end 145.5564 93.1054) (width 0.25) (layer "F.Cu") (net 5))
 (segment (start 144.3811 92.3255) (end 145.5564 92.3255) (width 0.25) (layer "F.Cu") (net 5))
 (segment (start 145.5564 93.1054) (end 145.5564 92.3255) (width 0.25) (layer "F.Cu") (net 5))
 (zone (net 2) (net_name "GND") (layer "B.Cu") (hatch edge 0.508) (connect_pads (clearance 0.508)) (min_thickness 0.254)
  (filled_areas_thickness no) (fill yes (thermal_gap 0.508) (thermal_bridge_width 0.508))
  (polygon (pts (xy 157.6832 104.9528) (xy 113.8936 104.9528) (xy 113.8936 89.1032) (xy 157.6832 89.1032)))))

